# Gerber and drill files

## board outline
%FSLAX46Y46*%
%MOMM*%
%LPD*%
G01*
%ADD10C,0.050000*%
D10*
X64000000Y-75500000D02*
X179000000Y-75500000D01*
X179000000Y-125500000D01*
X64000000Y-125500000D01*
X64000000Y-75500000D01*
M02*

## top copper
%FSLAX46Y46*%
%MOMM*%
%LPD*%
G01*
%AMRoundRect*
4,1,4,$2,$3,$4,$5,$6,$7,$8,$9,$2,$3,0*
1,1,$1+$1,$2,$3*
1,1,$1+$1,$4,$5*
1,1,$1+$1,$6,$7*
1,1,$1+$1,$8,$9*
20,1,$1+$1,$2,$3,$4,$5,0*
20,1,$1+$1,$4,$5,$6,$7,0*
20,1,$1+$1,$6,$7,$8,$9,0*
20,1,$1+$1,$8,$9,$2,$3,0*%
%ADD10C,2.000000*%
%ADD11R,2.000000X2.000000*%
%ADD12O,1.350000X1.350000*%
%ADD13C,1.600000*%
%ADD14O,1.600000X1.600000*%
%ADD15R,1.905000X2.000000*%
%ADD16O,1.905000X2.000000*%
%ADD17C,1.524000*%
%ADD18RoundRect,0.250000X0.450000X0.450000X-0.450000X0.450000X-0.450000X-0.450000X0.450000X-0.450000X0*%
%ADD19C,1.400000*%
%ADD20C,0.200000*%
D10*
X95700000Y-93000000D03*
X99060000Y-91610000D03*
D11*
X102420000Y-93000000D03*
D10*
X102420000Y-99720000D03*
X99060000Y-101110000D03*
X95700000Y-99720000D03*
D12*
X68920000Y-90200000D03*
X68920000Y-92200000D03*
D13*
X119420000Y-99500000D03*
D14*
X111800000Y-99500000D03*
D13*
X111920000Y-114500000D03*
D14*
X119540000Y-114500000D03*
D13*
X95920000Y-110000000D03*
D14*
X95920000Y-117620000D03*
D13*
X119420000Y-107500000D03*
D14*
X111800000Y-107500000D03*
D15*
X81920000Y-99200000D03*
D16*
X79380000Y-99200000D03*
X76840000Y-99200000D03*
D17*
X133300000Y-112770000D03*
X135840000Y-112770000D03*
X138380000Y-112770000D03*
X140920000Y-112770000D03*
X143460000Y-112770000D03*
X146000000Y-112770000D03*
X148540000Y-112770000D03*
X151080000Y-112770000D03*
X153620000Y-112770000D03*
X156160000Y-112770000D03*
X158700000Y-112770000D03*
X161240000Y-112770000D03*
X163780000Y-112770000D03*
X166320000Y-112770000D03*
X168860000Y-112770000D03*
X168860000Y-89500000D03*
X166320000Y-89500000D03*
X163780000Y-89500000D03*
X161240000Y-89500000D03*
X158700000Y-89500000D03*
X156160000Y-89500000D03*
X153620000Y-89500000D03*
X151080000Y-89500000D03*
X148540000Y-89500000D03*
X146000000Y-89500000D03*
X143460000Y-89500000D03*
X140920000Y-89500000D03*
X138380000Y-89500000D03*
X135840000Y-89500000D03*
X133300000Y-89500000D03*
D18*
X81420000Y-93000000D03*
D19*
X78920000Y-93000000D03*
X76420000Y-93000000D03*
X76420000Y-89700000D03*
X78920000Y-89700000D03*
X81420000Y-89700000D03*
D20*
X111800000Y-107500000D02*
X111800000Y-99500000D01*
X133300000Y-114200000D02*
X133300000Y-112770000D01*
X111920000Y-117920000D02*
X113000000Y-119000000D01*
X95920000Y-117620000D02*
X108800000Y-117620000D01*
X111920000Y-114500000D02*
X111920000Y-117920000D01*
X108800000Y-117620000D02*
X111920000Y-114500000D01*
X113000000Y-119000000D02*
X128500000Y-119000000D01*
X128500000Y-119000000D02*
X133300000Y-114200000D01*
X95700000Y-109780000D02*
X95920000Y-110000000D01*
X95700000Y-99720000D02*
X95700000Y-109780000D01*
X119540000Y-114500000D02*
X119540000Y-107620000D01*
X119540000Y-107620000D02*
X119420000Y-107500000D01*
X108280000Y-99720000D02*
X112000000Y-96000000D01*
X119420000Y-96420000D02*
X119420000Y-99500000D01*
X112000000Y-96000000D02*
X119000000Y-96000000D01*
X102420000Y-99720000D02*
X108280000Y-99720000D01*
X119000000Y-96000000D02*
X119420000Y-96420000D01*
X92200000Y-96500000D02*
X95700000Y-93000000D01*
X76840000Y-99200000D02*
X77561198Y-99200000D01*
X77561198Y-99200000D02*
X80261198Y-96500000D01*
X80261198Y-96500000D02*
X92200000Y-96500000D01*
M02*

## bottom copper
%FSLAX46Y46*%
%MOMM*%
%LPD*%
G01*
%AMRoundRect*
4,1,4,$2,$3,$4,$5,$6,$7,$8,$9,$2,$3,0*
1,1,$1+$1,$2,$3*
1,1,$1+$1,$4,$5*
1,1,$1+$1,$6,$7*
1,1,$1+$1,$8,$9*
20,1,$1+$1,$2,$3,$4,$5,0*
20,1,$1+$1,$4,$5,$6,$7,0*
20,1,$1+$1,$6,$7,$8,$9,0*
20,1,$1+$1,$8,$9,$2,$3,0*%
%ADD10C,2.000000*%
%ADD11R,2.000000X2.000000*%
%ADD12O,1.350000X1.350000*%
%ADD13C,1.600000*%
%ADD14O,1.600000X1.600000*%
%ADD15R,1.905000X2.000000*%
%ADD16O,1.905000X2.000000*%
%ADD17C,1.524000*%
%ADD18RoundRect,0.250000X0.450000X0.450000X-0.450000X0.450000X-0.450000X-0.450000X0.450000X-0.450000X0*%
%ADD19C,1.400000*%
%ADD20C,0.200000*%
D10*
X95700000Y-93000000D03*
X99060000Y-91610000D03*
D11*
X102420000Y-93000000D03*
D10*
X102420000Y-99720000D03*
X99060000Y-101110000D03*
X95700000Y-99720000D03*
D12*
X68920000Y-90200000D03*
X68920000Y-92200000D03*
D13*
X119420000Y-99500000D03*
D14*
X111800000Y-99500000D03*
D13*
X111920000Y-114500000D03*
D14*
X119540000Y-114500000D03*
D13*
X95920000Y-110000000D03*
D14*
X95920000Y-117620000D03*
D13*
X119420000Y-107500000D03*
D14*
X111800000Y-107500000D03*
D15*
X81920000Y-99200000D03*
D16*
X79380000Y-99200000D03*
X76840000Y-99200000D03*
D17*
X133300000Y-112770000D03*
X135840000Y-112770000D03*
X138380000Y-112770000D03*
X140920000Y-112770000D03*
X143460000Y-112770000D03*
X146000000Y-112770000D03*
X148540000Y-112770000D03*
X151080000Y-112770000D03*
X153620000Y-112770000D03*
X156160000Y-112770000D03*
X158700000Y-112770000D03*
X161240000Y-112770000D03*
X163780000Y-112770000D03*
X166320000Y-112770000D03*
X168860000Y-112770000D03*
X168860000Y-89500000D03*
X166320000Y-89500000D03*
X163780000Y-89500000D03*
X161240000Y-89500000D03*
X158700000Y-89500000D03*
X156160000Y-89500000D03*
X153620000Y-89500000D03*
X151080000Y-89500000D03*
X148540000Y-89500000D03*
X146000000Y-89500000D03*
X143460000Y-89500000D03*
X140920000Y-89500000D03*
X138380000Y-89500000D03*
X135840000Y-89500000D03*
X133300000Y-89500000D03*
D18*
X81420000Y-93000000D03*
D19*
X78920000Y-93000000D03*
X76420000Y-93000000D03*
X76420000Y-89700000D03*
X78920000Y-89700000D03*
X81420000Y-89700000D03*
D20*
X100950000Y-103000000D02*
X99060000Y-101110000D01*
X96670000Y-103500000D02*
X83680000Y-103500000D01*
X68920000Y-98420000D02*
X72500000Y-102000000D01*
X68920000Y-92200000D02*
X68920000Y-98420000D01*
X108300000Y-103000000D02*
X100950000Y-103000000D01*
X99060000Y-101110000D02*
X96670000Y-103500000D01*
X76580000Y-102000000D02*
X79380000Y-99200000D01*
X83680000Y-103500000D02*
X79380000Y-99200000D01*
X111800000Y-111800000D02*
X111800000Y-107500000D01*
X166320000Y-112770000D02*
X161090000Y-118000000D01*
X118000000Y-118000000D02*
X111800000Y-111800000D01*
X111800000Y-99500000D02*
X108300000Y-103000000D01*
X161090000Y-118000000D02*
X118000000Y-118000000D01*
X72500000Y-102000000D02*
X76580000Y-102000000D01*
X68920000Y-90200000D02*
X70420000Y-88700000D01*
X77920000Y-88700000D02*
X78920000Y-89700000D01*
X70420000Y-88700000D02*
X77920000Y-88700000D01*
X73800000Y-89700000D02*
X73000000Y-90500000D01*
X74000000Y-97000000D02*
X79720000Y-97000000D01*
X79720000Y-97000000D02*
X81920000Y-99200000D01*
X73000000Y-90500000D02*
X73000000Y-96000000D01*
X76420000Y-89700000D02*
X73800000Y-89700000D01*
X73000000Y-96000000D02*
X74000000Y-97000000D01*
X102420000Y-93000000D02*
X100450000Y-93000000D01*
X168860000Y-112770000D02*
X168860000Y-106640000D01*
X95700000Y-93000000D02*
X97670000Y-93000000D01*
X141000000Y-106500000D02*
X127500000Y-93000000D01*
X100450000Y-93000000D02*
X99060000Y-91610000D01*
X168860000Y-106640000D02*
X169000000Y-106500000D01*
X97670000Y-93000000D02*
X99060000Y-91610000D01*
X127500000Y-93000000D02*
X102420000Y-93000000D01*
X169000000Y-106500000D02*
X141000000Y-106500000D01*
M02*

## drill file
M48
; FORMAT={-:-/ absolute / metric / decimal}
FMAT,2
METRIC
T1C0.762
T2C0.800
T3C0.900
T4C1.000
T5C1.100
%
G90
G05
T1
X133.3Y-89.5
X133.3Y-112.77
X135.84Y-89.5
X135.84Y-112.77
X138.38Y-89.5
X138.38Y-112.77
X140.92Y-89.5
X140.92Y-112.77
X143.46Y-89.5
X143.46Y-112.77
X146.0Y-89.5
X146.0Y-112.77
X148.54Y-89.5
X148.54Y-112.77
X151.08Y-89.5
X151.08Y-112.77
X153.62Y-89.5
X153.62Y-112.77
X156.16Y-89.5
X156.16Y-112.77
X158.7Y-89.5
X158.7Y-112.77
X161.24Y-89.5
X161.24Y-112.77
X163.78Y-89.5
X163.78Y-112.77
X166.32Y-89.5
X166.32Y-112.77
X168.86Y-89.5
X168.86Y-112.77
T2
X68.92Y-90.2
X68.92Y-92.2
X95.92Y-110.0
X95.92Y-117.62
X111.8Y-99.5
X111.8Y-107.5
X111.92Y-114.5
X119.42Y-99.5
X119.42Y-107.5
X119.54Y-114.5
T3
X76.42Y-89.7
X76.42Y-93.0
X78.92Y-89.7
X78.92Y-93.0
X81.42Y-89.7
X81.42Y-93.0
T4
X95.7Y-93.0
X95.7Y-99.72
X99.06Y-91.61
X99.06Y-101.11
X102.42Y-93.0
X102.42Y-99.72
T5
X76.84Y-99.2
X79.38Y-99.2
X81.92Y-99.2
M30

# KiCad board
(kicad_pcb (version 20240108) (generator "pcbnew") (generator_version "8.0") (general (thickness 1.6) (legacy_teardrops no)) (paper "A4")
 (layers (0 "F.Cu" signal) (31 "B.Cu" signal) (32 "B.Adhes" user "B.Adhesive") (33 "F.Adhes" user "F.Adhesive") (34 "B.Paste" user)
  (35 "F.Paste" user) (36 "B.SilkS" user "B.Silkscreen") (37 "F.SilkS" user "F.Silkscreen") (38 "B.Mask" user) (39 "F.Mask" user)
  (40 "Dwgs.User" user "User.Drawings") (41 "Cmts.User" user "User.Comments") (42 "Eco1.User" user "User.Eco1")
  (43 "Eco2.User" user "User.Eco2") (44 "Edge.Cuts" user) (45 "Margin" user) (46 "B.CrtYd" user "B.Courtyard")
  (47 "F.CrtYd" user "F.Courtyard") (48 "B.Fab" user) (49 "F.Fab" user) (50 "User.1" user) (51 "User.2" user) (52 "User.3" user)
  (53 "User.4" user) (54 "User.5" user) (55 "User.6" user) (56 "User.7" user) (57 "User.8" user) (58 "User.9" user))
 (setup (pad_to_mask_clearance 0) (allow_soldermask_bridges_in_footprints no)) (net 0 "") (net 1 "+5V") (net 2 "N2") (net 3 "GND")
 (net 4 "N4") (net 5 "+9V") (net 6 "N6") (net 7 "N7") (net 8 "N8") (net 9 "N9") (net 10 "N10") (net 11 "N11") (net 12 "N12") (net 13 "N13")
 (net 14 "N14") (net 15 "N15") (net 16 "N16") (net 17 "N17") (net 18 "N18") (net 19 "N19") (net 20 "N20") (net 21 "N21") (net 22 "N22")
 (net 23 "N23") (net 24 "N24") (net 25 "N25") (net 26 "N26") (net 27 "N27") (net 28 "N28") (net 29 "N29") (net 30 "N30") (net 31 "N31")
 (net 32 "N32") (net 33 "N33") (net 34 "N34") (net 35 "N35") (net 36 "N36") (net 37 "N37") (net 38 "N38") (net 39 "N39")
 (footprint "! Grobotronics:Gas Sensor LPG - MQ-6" (layer "F.Cu") (at 98.999941 96.406859)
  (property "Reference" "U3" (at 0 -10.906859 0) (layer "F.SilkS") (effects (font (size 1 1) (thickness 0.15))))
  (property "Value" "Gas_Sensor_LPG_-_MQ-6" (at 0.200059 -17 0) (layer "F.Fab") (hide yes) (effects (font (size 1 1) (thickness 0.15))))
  (pad "1" thru_hole circle (at -3.299941 -3.406859) (size 2 2) (drill 1) (layers "*.Cu" "*.Mask") (remove_unused_layers no) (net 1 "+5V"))
  (pad "2" thru_hole circle (at 0.060059 -4.796859 270) (size 2 2) (drill 1) (layers "*.Cu" "*.Mask") (remove_unused_layers no)
   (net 1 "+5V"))
  (pad "3" thru_hole rect (at 3.420059 -3.406859 270) (size 2 2) (drill 1) (layers "*.Cu" "*.Mask") (remove_unused_layers no) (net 1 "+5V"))
  (pad "4" thru_hole circle (at 3.420059 3.313141 180) (size 2 2) (drill 1) (layers "*.Cu" "*.Mask") (remove_unused_layers no) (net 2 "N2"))
  (pad "5" thru_hole circle (at 0.060059 4.703141 270) (size 2 2) (drill 1) (layers "*.Cu" "*.Mask") (remove_unused_layers no) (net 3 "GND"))
  (pad "6" thru_hole circle (at -3.299941 3.313141 90) (size 2 2) (drill 1) (layers "*.Cu" "*.Mask") (remove_unused_layers no) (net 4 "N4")))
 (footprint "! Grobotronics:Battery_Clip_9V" (layer "F.Cu") (at 68.92 90.7)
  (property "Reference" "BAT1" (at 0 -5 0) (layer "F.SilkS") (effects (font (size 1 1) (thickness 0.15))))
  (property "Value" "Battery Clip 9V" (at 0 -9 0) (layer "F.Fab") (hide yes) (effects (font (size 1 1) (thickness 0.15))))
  (pad "+" thru_hole oval (at 0 -0.5) (size 1.35 1.35) (drill 0.8) (layers "*.Cu" "*.Mask") (remove_unused_layers no) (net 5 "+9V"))
  (pad "-" thru_hole oval (at 0 1.5) (size 1.35 1.35) (drill 0.8) (layers "*.Cu" "*.Mask") (remove_unused_layers no) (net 3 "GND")))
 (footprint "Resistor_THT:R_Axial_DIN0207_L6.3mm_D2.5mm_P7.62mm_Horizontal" (layer "F.Cu") (at 119.42 99.5 180)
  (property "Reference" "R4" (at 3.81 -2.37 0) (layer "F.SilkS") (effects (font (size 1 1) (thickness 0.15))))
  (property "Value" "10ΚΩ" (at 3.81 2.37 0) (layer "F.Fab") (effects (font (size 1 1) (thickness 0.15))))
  (pad "1" thru_hole circle (at 0 0 180) (size 1.6 1.6) (drill 0.8) (layers "*.Cu" "*.Mask") (remove_unused_layers no) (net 2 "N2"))
  (pad "2" thru_hole oval (at 7.62 0 180) (size 1.6 1.6) (drill 0.8) (layers "*.Cu" "*.Mask") (remove_unused_layers no) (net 3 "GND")))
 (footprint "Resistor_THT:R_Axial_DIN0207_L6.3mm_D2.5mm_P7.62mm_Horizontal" (layer "F.Cu") (at 111.92 114.5)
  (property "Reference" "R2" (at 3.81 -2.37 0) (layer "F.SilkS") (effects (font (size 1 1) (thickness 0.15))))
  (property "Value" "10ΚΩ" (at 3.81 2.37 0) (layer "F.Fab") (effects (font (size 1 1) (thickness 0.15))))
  (pad "1" thru_hole circle (at 0 0) (size 1.6 1.6) (drill 0.8) (layers "*.Cu" "*.Mask") (remove_unused_layers no) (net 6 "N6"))
  (pad "2" thru_hole oval (at 7.62 0) (size 1.6 1.6) (drill 0.8) (layers "*.Cu" "*.Mask") (remove_unused_layers no) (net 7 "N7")))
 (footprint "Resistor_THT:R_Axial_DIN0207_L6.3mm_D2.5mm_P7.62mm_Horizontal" (layer "F.Cu") (at 95.92 110 -90)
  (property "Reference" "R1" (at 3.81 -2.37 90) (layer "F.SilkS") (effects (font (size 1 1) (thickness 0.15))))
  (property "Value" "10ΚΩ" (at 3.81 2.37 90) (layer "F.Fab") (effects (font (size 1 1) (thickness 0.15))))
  (pad "1" thru_hole circle (at 0 0 270) (size 1.6 1.6) (drill 0.8) (layers "*.Cu" "*.Mask") (remove_unused_layers no) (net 4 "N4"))
  (pad "2" thru_hole oval (at 7.62 0 270) (size 1.6 1.6) (drill 0.8) (layers "*.Cu" "*.Mask") (remove_unused_layers no) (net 6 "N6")))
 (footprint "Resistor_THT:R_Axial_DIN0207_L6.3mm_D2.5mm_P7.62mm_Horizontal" (layer "F.Cu") (at 119.42 107.5 180)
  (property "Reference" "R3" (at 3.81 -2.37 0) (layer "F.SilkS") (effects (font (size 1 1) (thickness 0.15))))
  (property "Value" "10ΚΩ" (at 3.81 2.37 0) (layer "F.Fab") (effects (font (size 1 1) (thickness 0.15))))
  (pad "1" thru_hole circle (at 0 0 180) (size 1.6 1.6) (drill 0.8) (layers "*.Cu" "*.Mask") (remove_unused_layers no) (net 7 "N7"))
  (pad "2" thru_hole oval (at 7.62 0 180) (size 1.6 1.6) (drill 0.8) (layers "*.Cu" "*.Mask") (remove_unused_layers no) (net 3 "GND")))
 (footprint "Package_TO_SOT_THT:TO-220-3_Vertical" (layer "F.Cu") (at 81.92 99.2 180)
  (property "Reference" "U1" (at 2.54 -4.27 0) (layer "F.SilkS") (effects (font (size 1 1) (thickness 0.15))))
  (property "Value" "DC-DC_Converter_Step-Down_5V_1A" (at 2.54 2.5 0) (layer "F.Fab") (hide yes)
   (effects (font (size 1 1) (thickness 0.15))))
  (pad "1" thru_hole rect (at 0 0 180) (size 1.905 2) (drill 1.1) (layers "*.Cu" "*.Mask") (remove_unused_layers no) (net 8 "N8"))
  (pad "2" thru_hole oval (at 2.54 0 180) (size 1.905 2) (drill 1.1) (layers "*.Cu" "*.Mask") (remove_unused_layers no) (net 3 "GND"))
  (pad "3" thru_hole oval (at 5.08 0 180) (size 1.905 2) (drill 1.1) (layers "*.Cu" "*.Mask") (remove_unused_layers no) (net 1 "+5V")))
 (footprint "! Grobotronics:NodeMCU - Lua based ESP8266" (layer "F.Cu") (at 151.08 101.27 90)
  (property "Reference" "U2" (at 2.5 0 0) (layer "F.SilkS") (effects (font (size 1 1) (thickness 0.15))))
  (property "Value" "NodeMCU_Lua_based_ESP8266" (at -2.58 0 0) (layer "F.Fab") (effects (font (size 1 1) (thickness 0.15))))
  (pad "1" thru_hole circle (at -11.5 -17.78 90) (size 1.524 1.524) (drill 0.762) (layers "*.Cu" "*.Mask") (remove_unused_layers no)
   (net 6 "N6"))
  (pad "2" thru_hole circle (at -11.5 -15.24 90) (size 1.524 1.524) (drill 0.762) (layers "*.Cu" "*.Mask") (remove_unused_layers no)
   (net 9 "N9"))
  (pad "3" thru_hole circle (at -11.5 -12.7 90) (size 1.524 1.524) (drill 0.762) (layers "*.Cu" "*.Mask") (remove_unused_layers no)
   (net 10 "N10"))
  (pad "4" thru_hole circle (at -11.5 -10.16 90) (size 1.524 1.524) (drill 0.762) (layers "*.Cu" "*.Mask") (remove_unused_layers no)
   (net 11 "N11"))
  (pad "5" thru_hole circle (at -11.5 -7.62 90) (size 1.524 1.524) (drill 0.762) (layers "*.Cu" "*.Mask") (remove_unused_layers no)
   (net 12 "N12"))
  (pad "6" thru_hole circle (at -11.5 -5.08 90) (size 1.524 1.524) (drill 0.762) (layers "*.Cu" "*.Mask") (remove_unused_layers no)
   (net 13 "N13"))
  (pad "7" thru_hole circle (at -11.5 -2.54 90) (size 1.524 1.524) (drill 0.762) (layers "*.Cu" "*.Mask") (remove_unused_layers no)
   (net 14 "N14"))
  (pad "8" thru_hole circle (at -11.5 0 90) (size 1.524 1.524) (drill 0.762) (layers "*.Cu" "*.Mask") (remove_unused_layers no)
   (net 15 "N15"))
  (pad "9" thru_hole circle (at -11.5 2.54 90) (size 1.524 1.524) (drill 0.762) (layers "*.Cu" "*.Mask") (remove_unused_layers no)
   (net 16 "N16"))
  (pad "10" thru_hole circle (at -11.5 5.08 90) (size 1.524 1.524) (drill 0.762) (layers "*.Cu" "*.Mask") (remove_unused_layers no)
   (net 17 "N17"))
  (pad "11" thru_hole circle (at -11.5 7.62 90) (size 1.524 1.524) (drill 0.762) (layers "*.Cu" "*.Mask") (remove_unused_layers no)
   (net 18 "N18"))
  (pad "12" thru_hole circle (at -11.5 10.16 90) (size 1.524 1.524) (drill 0.762) (layers "*.Cu" "*.Mask") (remove_unused_layers no)
   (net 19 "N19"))
  (pad "13" thru_hole circle (at -11.5 12.7 90) (size 1.524 1.524) (drill 0.762) (layers "*.Cu" "*.Mask") (remove_unused_layers no)
   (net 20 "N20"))
  (pad "14" thru_hole circle (at -11.5 15.24 90) (size 1.524 1.524) (drill 0.762) (layers "*.Cu" "*.Mask") (remove_unused_layers no)
   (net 3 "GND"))
  (pad "15" thru_hole circle (at -11.5 17.78 90) (size 1.524 1.524) (drill 0.762) (layers "*.Cu" "*.Mask") (remove_unused_layers no)
   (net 1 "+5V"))
  (pad "16" thru_hole circle (at 11.77 17.78 90) (size 1.524 1.524) (drill 0.762) (layers "*.Cu" "*.Mask") (remove_unused_layers no)
   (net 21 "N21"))
  (pad "17" thru_hole circle (at 11.77 15.24 90) (size 1.524 1.524) (drill 0.762) (layers "*.Cu" "*.Mask") (remove_unused_layers no)
   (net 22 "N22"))
  (pad "18" thru_hole circle (at 11.77 12.7 90) (size 1.524 1.524) (drill 0.762) (layers "*.Cu" "*.Mask") (remove_unused_layers no)
   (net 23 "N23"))
  (pad "19" thru_hole circle (at 11.77 10.16 90) (size 1.524 1.524) (drill 0.762) (layers "*.Cu" "*.Mask") (remove_unused_layers no)
   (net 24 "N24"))
  (pad "20" thru_hole circle (at 11.77 7.62 90) (size 1.524 1.524) (drill 0.762) (layers "*.Cu" "*.Mask") (remove_unused_layers no)
   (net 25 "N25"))
  (pad "21" thru_hole circle (at 11.77 5.08 90) (size 1.524 1.524) (drill 0.762) (layers "*.Cu" "*.Mask") (remove_unused_layers no)
   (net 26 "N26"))
  (pad "22" thru_hole circle (at 11.77 2.54 90) (size 1.524 1.524) (drill 0.762) (layers "*.Cu" "*.Mask") (remove_unused_layers no)
   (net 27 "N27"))
  (pad "23" thru_hole circle (at 11.77 0 90) (size 1.524 1.524) (drill 0.762) (layers "*.Cu" "*.Mask") (remove_unused_layers no)
   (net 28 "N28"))
  (pad "24" thru_hole circle (at 11.77 -2.54 90) (size 1.524 1.524) (drill 0.762) (layers "*.Cu" "*.Mask") (remove_unused_layers no)
   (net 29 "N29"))
  (pad "25" thru_hole circle (at 11.77 -5.08 90) (size 1.524 1.524) (drill 0.762) (layers "*.Cu" "*.Mask") (remove_unused_layers no)
   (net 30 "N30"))
  (pad "26" thru_hole circle (at 11.77 -7.62 90) (size 1.524 1.524) (drill 0.762) (layers "*.Cu" "*.Mask") (remove_unused_layers no)
   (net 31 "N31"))
  (pad "27" thru_hole circle (at 11.77 -10.16 90) (size 1.524 1.524) (drill 0.762) (layers "*.Cu" "*.Mask") (remove_unused_layers no)
   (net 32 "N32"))
  (pad "28" thru_hole circle (at 11.77 -12.7 90) (size 1.524 1.524) (drill 0.762) (layers "*.Cu" "*.Mask") (remove_unused_layers no)
   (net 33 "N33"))
  (pad "29" thru_hole circle (at 11.77 -15.24 90) (size 1.524 1.524) (drill 0.762) (layers "*.Cu" "*.Mask") (remove_unused_layers no)
   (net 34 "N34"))
  (pad "30" thru_hole circle (at 11.77 -17.78 90) (size 1.524 1.524) (drill 0.762) (layers "*.Cu" "*.Mask") (remove_unused_layers no)
   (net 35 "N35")))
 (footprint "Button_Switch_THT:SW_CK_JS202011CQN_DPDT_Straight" (layer "F.Cu") (at 81.42 93 180)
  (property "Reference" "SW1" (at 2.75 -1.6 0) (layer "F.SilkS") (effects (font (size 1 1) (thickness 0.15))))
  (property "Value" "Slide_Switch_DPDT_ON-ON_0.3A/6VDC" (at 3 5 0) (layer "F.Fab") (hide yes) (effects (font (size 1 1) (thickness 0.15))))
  (pad "1" thru_hole roundrect (at 0 0 180) (size 1.4 1.4) (drill 0.9) (layers "*.Cu" "*.Mask") (remove_unused_layers no)
   (roundrect_rratio 0.1785714286) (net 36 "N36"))
  (pad "2" thru_hole circle (at 2.5 0 180) (size 1.4 1.4) (drill 0.9) (layers "*.Cu" "*.Mask") (remove_unused_layers no) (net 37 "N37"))
  (pad "3" thru_hole circle (at 5 0 180) (size 1.4 1.4) (drill 0.9) (layers "*.Cu" "*.Mask") (remove_unused_layers no) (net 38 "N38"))
  (pad "4" thru_hole circle (at 5 3.3 180) (size 1.4 1.4) (drill 0.9) (layers "*.Cu" "*.Mask") (remove_unused_layers no) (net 8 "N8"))
  (pad "5" thru_hole circle (at 2.5 3.3 180) (size 1.4 1.4) (drill 0.9) (layers "*.Cu" "*.Mask") (remove_unused_layers no) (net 5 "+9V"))
  (pad "6" thru_hole circle (at 0 3.3 180) (size 1.4 1.4) (drill 0.9) (layers "*.Cu" "*.Mask") (remove_unused_layers no) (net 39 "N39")))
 (gr_rect (start 64 75.5) (end 179 125.5) (stroke (width 0.05) (type default)) (fill none) (layer "Edge.Cuts"))
 (segment (start 111.8 107.5) (end 111.8 99.5) (width 0.2) (layer "F.Cu") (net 3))
 (segment (start 100.95 103) (end 99.06 101.11) (width 0.2) (layer "B.Cu") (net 3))
 (segment (start 96.67 103.5) (end 83.68 103.5) (width 0.2) (layer "B.Cu") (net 3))
 (segment (start 68.92 98.42) (end 72.5 102) (width 0.2) (layer "B.Cu") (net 3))
 (segment (start 68.92 92.2) (end 68.92 98.42) (width 0.2) (layer "B.Cu") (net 3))
 (segment (start 108.3 103) (end 100.95 103) (width 0.2) (layer "B.Cu") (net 3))
 (segment (start 99.06 101.11) (end 96.67 103.5) (width 0.2) (layer "B.Cu") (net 3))
 (segment (start 76.58 102) (end 79.38 99.2) (width 0.2) (layer "B.Cu") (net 3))
 (segment (start 83.68 103.5) (end 79.38 99.2) (width 0.2) (layer "B.Cu") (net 3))
 (segment (start 111.8 111.8) (end 111.8 107.5) (width 0.2) (layer "B.Cu") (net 3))
 (segment (start 166.32 112.77) (end 161.09 118) (width 0.2) (layer "B.Cu") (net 3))
 (segment (start 118 118) (end 111.8 111.8) (width 0.2) (layer "B.Cu") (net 3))
 (segment (start 111.8 99.5) (end 108.3 103) (width 0.2) (layer "B.Cu") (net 3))
 (segment (start 161.09 118) (end 118 118) (width 0.2) (layer "B.Cu") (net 3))
 (segment (start 72.5 102) (end 76.58 102) (width 0.2) (layer "B.Cu") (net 3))
 (segment (start 68.92 90.2) (end 70.42 88.7) (width 0.2) (layer "B.Cu") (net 5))
 (segment (start 77.92 88.7) (end 78.92 89.7) (width 0.2) (layer "B.Cu") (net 5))
 (segment (start 70.42 88.7) (end 77.92 88.7) (width 0.2) (layer "B.Cu") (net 5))
 (segment (start 133.3 114.2) (end 133.3 112.77) (width 0.2) (layer "F.Cu") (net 6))
 (segment (start 111.92 117.92) (end 113 119) (width 0.2) (layer "F.Cu") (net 6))
 (segment (start 95.92 117.62) (end 108.8 117.62) (width 0.2) (layer "F.Cu") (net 6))
 (segment (start 111.92 114.5) (end 111.92 117.92) (width 0.2) (layer "F.Cu") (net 6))
 (segment (start 108.8 117.62) (end 111.92 114.5) (width 0.2) (layer "F.Cu") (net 6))
 (segment (start 113 119) (end 128.5 119) (width 0.2) (layer "F.Cu") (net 6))
 (segment (start 128.5 119) (end 133.3 114.2) (width 0.2) (layer "F.Cu") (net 6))
 (segment (start 95.7 109.78) (end 95.92 110) (width 0.2) (layer "F.Cu") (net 4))
 (segment (start 95.7 99.72) (end 95.7 109.78) (width 0.2) (layer "F.Cu") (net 4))
 (segment (start 119.54 114.5) (end 119.54 107.62) (width 0.2) (layer "F.Cu") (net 7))
 (segment (start 119.54 107.62) (end 119.42 107.5) (width 0.2) (layer "F.Cu") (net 7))
 (segment (start 108.28 99.72) (end 112 96) (width 0.2) (layer "F.Cu") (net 2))
 (segment (start 119.42 96.42) (end 119.42 99.5) (width 0.2) (layer "F.Cu") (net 2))
 (segment (start 112 96) (end 119 96) (width 0.2) (layer "F.Cu") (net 2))
 (segment (start 102.42 99.72) (end 108.28 99.72) (width 0.2) (layer "F.Cu") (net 2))
 (segment (start 119 96) (end 119.42 96.42) (width 0.2) (layer "F.Cu") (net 2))
 (segment (start 73.8 89.7) (end 73 90.5) (width 0.2) (layer "B.Cu") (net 8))
 (segment (start 74 97) (end 79.72 97) (width 0.2) (layer "B.Cu") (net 8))
 (segment (start 79.72 97) (end 81.92 99.2) (width 0.2) (layer "B.Cu") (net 8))
 (segment (start 73 90.5) (end 73 96) (width 0.2) (layer "B.Cu") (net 8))
 (segment (start 76.42 89.7) (end 73.8 89.7) (width 0.2) (layer "B.Cu") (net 8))
 (segment (start 73 96) (end 74 97) (width 0.2) (layer "B.Cu") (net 8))
 (segment (start 92.2 96.5) (end 95.7 93) (width 0.2) (layer "F.Cu") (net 1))
 (segment (start 76.84 99.2) (end 77.561198 99.2) (width 0.2) (layer "F.Cu") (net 1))
 (segment (start 77.561198 99.2) (end 80.261198 96.5) (width 0.2) (layer "F.Cu") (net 1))
 (segment (start 80.261198 96.5) (end 92.2 96.5) (width 0.2) (layer "F.Cu") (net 1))
 (segment (start 102.42 93) (end 100.45 93) (width 0.2) (layer "B.Cu") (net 1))
 (segment (start 168.86 112.77) (end 168.86 106.64) (width 0.2) (layer "B.Cu") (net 1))
 (segment (start 95.7 93) (end 97.67 93) (width 0.2) (layer "B.Cu") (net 1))
 (segment (start 141 106.5) (end 127.5 93) (width 0.2) (layer "B.Cu") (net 1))
 (segment (start 100.45 93) (end 99.06 91.61) (width 0.2) (layer "B.Cu") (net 1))
 (segment (start 168.86 106.64) (end 169 106.5) (width 0.2) (layer "B.Cu") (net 1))
 (segment (start 97.67 93) (end 99.06 91.61) (width 0.2) (layer "B.Cu") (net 1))
 (segment (start 127.5 93) (end 102.42 93) (width 0.2) (layer "B.Cu") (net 1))
 (segment (start 169 106.5) (end 141 106.5) (width 0.2) (layer "B.Cu") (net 1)))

